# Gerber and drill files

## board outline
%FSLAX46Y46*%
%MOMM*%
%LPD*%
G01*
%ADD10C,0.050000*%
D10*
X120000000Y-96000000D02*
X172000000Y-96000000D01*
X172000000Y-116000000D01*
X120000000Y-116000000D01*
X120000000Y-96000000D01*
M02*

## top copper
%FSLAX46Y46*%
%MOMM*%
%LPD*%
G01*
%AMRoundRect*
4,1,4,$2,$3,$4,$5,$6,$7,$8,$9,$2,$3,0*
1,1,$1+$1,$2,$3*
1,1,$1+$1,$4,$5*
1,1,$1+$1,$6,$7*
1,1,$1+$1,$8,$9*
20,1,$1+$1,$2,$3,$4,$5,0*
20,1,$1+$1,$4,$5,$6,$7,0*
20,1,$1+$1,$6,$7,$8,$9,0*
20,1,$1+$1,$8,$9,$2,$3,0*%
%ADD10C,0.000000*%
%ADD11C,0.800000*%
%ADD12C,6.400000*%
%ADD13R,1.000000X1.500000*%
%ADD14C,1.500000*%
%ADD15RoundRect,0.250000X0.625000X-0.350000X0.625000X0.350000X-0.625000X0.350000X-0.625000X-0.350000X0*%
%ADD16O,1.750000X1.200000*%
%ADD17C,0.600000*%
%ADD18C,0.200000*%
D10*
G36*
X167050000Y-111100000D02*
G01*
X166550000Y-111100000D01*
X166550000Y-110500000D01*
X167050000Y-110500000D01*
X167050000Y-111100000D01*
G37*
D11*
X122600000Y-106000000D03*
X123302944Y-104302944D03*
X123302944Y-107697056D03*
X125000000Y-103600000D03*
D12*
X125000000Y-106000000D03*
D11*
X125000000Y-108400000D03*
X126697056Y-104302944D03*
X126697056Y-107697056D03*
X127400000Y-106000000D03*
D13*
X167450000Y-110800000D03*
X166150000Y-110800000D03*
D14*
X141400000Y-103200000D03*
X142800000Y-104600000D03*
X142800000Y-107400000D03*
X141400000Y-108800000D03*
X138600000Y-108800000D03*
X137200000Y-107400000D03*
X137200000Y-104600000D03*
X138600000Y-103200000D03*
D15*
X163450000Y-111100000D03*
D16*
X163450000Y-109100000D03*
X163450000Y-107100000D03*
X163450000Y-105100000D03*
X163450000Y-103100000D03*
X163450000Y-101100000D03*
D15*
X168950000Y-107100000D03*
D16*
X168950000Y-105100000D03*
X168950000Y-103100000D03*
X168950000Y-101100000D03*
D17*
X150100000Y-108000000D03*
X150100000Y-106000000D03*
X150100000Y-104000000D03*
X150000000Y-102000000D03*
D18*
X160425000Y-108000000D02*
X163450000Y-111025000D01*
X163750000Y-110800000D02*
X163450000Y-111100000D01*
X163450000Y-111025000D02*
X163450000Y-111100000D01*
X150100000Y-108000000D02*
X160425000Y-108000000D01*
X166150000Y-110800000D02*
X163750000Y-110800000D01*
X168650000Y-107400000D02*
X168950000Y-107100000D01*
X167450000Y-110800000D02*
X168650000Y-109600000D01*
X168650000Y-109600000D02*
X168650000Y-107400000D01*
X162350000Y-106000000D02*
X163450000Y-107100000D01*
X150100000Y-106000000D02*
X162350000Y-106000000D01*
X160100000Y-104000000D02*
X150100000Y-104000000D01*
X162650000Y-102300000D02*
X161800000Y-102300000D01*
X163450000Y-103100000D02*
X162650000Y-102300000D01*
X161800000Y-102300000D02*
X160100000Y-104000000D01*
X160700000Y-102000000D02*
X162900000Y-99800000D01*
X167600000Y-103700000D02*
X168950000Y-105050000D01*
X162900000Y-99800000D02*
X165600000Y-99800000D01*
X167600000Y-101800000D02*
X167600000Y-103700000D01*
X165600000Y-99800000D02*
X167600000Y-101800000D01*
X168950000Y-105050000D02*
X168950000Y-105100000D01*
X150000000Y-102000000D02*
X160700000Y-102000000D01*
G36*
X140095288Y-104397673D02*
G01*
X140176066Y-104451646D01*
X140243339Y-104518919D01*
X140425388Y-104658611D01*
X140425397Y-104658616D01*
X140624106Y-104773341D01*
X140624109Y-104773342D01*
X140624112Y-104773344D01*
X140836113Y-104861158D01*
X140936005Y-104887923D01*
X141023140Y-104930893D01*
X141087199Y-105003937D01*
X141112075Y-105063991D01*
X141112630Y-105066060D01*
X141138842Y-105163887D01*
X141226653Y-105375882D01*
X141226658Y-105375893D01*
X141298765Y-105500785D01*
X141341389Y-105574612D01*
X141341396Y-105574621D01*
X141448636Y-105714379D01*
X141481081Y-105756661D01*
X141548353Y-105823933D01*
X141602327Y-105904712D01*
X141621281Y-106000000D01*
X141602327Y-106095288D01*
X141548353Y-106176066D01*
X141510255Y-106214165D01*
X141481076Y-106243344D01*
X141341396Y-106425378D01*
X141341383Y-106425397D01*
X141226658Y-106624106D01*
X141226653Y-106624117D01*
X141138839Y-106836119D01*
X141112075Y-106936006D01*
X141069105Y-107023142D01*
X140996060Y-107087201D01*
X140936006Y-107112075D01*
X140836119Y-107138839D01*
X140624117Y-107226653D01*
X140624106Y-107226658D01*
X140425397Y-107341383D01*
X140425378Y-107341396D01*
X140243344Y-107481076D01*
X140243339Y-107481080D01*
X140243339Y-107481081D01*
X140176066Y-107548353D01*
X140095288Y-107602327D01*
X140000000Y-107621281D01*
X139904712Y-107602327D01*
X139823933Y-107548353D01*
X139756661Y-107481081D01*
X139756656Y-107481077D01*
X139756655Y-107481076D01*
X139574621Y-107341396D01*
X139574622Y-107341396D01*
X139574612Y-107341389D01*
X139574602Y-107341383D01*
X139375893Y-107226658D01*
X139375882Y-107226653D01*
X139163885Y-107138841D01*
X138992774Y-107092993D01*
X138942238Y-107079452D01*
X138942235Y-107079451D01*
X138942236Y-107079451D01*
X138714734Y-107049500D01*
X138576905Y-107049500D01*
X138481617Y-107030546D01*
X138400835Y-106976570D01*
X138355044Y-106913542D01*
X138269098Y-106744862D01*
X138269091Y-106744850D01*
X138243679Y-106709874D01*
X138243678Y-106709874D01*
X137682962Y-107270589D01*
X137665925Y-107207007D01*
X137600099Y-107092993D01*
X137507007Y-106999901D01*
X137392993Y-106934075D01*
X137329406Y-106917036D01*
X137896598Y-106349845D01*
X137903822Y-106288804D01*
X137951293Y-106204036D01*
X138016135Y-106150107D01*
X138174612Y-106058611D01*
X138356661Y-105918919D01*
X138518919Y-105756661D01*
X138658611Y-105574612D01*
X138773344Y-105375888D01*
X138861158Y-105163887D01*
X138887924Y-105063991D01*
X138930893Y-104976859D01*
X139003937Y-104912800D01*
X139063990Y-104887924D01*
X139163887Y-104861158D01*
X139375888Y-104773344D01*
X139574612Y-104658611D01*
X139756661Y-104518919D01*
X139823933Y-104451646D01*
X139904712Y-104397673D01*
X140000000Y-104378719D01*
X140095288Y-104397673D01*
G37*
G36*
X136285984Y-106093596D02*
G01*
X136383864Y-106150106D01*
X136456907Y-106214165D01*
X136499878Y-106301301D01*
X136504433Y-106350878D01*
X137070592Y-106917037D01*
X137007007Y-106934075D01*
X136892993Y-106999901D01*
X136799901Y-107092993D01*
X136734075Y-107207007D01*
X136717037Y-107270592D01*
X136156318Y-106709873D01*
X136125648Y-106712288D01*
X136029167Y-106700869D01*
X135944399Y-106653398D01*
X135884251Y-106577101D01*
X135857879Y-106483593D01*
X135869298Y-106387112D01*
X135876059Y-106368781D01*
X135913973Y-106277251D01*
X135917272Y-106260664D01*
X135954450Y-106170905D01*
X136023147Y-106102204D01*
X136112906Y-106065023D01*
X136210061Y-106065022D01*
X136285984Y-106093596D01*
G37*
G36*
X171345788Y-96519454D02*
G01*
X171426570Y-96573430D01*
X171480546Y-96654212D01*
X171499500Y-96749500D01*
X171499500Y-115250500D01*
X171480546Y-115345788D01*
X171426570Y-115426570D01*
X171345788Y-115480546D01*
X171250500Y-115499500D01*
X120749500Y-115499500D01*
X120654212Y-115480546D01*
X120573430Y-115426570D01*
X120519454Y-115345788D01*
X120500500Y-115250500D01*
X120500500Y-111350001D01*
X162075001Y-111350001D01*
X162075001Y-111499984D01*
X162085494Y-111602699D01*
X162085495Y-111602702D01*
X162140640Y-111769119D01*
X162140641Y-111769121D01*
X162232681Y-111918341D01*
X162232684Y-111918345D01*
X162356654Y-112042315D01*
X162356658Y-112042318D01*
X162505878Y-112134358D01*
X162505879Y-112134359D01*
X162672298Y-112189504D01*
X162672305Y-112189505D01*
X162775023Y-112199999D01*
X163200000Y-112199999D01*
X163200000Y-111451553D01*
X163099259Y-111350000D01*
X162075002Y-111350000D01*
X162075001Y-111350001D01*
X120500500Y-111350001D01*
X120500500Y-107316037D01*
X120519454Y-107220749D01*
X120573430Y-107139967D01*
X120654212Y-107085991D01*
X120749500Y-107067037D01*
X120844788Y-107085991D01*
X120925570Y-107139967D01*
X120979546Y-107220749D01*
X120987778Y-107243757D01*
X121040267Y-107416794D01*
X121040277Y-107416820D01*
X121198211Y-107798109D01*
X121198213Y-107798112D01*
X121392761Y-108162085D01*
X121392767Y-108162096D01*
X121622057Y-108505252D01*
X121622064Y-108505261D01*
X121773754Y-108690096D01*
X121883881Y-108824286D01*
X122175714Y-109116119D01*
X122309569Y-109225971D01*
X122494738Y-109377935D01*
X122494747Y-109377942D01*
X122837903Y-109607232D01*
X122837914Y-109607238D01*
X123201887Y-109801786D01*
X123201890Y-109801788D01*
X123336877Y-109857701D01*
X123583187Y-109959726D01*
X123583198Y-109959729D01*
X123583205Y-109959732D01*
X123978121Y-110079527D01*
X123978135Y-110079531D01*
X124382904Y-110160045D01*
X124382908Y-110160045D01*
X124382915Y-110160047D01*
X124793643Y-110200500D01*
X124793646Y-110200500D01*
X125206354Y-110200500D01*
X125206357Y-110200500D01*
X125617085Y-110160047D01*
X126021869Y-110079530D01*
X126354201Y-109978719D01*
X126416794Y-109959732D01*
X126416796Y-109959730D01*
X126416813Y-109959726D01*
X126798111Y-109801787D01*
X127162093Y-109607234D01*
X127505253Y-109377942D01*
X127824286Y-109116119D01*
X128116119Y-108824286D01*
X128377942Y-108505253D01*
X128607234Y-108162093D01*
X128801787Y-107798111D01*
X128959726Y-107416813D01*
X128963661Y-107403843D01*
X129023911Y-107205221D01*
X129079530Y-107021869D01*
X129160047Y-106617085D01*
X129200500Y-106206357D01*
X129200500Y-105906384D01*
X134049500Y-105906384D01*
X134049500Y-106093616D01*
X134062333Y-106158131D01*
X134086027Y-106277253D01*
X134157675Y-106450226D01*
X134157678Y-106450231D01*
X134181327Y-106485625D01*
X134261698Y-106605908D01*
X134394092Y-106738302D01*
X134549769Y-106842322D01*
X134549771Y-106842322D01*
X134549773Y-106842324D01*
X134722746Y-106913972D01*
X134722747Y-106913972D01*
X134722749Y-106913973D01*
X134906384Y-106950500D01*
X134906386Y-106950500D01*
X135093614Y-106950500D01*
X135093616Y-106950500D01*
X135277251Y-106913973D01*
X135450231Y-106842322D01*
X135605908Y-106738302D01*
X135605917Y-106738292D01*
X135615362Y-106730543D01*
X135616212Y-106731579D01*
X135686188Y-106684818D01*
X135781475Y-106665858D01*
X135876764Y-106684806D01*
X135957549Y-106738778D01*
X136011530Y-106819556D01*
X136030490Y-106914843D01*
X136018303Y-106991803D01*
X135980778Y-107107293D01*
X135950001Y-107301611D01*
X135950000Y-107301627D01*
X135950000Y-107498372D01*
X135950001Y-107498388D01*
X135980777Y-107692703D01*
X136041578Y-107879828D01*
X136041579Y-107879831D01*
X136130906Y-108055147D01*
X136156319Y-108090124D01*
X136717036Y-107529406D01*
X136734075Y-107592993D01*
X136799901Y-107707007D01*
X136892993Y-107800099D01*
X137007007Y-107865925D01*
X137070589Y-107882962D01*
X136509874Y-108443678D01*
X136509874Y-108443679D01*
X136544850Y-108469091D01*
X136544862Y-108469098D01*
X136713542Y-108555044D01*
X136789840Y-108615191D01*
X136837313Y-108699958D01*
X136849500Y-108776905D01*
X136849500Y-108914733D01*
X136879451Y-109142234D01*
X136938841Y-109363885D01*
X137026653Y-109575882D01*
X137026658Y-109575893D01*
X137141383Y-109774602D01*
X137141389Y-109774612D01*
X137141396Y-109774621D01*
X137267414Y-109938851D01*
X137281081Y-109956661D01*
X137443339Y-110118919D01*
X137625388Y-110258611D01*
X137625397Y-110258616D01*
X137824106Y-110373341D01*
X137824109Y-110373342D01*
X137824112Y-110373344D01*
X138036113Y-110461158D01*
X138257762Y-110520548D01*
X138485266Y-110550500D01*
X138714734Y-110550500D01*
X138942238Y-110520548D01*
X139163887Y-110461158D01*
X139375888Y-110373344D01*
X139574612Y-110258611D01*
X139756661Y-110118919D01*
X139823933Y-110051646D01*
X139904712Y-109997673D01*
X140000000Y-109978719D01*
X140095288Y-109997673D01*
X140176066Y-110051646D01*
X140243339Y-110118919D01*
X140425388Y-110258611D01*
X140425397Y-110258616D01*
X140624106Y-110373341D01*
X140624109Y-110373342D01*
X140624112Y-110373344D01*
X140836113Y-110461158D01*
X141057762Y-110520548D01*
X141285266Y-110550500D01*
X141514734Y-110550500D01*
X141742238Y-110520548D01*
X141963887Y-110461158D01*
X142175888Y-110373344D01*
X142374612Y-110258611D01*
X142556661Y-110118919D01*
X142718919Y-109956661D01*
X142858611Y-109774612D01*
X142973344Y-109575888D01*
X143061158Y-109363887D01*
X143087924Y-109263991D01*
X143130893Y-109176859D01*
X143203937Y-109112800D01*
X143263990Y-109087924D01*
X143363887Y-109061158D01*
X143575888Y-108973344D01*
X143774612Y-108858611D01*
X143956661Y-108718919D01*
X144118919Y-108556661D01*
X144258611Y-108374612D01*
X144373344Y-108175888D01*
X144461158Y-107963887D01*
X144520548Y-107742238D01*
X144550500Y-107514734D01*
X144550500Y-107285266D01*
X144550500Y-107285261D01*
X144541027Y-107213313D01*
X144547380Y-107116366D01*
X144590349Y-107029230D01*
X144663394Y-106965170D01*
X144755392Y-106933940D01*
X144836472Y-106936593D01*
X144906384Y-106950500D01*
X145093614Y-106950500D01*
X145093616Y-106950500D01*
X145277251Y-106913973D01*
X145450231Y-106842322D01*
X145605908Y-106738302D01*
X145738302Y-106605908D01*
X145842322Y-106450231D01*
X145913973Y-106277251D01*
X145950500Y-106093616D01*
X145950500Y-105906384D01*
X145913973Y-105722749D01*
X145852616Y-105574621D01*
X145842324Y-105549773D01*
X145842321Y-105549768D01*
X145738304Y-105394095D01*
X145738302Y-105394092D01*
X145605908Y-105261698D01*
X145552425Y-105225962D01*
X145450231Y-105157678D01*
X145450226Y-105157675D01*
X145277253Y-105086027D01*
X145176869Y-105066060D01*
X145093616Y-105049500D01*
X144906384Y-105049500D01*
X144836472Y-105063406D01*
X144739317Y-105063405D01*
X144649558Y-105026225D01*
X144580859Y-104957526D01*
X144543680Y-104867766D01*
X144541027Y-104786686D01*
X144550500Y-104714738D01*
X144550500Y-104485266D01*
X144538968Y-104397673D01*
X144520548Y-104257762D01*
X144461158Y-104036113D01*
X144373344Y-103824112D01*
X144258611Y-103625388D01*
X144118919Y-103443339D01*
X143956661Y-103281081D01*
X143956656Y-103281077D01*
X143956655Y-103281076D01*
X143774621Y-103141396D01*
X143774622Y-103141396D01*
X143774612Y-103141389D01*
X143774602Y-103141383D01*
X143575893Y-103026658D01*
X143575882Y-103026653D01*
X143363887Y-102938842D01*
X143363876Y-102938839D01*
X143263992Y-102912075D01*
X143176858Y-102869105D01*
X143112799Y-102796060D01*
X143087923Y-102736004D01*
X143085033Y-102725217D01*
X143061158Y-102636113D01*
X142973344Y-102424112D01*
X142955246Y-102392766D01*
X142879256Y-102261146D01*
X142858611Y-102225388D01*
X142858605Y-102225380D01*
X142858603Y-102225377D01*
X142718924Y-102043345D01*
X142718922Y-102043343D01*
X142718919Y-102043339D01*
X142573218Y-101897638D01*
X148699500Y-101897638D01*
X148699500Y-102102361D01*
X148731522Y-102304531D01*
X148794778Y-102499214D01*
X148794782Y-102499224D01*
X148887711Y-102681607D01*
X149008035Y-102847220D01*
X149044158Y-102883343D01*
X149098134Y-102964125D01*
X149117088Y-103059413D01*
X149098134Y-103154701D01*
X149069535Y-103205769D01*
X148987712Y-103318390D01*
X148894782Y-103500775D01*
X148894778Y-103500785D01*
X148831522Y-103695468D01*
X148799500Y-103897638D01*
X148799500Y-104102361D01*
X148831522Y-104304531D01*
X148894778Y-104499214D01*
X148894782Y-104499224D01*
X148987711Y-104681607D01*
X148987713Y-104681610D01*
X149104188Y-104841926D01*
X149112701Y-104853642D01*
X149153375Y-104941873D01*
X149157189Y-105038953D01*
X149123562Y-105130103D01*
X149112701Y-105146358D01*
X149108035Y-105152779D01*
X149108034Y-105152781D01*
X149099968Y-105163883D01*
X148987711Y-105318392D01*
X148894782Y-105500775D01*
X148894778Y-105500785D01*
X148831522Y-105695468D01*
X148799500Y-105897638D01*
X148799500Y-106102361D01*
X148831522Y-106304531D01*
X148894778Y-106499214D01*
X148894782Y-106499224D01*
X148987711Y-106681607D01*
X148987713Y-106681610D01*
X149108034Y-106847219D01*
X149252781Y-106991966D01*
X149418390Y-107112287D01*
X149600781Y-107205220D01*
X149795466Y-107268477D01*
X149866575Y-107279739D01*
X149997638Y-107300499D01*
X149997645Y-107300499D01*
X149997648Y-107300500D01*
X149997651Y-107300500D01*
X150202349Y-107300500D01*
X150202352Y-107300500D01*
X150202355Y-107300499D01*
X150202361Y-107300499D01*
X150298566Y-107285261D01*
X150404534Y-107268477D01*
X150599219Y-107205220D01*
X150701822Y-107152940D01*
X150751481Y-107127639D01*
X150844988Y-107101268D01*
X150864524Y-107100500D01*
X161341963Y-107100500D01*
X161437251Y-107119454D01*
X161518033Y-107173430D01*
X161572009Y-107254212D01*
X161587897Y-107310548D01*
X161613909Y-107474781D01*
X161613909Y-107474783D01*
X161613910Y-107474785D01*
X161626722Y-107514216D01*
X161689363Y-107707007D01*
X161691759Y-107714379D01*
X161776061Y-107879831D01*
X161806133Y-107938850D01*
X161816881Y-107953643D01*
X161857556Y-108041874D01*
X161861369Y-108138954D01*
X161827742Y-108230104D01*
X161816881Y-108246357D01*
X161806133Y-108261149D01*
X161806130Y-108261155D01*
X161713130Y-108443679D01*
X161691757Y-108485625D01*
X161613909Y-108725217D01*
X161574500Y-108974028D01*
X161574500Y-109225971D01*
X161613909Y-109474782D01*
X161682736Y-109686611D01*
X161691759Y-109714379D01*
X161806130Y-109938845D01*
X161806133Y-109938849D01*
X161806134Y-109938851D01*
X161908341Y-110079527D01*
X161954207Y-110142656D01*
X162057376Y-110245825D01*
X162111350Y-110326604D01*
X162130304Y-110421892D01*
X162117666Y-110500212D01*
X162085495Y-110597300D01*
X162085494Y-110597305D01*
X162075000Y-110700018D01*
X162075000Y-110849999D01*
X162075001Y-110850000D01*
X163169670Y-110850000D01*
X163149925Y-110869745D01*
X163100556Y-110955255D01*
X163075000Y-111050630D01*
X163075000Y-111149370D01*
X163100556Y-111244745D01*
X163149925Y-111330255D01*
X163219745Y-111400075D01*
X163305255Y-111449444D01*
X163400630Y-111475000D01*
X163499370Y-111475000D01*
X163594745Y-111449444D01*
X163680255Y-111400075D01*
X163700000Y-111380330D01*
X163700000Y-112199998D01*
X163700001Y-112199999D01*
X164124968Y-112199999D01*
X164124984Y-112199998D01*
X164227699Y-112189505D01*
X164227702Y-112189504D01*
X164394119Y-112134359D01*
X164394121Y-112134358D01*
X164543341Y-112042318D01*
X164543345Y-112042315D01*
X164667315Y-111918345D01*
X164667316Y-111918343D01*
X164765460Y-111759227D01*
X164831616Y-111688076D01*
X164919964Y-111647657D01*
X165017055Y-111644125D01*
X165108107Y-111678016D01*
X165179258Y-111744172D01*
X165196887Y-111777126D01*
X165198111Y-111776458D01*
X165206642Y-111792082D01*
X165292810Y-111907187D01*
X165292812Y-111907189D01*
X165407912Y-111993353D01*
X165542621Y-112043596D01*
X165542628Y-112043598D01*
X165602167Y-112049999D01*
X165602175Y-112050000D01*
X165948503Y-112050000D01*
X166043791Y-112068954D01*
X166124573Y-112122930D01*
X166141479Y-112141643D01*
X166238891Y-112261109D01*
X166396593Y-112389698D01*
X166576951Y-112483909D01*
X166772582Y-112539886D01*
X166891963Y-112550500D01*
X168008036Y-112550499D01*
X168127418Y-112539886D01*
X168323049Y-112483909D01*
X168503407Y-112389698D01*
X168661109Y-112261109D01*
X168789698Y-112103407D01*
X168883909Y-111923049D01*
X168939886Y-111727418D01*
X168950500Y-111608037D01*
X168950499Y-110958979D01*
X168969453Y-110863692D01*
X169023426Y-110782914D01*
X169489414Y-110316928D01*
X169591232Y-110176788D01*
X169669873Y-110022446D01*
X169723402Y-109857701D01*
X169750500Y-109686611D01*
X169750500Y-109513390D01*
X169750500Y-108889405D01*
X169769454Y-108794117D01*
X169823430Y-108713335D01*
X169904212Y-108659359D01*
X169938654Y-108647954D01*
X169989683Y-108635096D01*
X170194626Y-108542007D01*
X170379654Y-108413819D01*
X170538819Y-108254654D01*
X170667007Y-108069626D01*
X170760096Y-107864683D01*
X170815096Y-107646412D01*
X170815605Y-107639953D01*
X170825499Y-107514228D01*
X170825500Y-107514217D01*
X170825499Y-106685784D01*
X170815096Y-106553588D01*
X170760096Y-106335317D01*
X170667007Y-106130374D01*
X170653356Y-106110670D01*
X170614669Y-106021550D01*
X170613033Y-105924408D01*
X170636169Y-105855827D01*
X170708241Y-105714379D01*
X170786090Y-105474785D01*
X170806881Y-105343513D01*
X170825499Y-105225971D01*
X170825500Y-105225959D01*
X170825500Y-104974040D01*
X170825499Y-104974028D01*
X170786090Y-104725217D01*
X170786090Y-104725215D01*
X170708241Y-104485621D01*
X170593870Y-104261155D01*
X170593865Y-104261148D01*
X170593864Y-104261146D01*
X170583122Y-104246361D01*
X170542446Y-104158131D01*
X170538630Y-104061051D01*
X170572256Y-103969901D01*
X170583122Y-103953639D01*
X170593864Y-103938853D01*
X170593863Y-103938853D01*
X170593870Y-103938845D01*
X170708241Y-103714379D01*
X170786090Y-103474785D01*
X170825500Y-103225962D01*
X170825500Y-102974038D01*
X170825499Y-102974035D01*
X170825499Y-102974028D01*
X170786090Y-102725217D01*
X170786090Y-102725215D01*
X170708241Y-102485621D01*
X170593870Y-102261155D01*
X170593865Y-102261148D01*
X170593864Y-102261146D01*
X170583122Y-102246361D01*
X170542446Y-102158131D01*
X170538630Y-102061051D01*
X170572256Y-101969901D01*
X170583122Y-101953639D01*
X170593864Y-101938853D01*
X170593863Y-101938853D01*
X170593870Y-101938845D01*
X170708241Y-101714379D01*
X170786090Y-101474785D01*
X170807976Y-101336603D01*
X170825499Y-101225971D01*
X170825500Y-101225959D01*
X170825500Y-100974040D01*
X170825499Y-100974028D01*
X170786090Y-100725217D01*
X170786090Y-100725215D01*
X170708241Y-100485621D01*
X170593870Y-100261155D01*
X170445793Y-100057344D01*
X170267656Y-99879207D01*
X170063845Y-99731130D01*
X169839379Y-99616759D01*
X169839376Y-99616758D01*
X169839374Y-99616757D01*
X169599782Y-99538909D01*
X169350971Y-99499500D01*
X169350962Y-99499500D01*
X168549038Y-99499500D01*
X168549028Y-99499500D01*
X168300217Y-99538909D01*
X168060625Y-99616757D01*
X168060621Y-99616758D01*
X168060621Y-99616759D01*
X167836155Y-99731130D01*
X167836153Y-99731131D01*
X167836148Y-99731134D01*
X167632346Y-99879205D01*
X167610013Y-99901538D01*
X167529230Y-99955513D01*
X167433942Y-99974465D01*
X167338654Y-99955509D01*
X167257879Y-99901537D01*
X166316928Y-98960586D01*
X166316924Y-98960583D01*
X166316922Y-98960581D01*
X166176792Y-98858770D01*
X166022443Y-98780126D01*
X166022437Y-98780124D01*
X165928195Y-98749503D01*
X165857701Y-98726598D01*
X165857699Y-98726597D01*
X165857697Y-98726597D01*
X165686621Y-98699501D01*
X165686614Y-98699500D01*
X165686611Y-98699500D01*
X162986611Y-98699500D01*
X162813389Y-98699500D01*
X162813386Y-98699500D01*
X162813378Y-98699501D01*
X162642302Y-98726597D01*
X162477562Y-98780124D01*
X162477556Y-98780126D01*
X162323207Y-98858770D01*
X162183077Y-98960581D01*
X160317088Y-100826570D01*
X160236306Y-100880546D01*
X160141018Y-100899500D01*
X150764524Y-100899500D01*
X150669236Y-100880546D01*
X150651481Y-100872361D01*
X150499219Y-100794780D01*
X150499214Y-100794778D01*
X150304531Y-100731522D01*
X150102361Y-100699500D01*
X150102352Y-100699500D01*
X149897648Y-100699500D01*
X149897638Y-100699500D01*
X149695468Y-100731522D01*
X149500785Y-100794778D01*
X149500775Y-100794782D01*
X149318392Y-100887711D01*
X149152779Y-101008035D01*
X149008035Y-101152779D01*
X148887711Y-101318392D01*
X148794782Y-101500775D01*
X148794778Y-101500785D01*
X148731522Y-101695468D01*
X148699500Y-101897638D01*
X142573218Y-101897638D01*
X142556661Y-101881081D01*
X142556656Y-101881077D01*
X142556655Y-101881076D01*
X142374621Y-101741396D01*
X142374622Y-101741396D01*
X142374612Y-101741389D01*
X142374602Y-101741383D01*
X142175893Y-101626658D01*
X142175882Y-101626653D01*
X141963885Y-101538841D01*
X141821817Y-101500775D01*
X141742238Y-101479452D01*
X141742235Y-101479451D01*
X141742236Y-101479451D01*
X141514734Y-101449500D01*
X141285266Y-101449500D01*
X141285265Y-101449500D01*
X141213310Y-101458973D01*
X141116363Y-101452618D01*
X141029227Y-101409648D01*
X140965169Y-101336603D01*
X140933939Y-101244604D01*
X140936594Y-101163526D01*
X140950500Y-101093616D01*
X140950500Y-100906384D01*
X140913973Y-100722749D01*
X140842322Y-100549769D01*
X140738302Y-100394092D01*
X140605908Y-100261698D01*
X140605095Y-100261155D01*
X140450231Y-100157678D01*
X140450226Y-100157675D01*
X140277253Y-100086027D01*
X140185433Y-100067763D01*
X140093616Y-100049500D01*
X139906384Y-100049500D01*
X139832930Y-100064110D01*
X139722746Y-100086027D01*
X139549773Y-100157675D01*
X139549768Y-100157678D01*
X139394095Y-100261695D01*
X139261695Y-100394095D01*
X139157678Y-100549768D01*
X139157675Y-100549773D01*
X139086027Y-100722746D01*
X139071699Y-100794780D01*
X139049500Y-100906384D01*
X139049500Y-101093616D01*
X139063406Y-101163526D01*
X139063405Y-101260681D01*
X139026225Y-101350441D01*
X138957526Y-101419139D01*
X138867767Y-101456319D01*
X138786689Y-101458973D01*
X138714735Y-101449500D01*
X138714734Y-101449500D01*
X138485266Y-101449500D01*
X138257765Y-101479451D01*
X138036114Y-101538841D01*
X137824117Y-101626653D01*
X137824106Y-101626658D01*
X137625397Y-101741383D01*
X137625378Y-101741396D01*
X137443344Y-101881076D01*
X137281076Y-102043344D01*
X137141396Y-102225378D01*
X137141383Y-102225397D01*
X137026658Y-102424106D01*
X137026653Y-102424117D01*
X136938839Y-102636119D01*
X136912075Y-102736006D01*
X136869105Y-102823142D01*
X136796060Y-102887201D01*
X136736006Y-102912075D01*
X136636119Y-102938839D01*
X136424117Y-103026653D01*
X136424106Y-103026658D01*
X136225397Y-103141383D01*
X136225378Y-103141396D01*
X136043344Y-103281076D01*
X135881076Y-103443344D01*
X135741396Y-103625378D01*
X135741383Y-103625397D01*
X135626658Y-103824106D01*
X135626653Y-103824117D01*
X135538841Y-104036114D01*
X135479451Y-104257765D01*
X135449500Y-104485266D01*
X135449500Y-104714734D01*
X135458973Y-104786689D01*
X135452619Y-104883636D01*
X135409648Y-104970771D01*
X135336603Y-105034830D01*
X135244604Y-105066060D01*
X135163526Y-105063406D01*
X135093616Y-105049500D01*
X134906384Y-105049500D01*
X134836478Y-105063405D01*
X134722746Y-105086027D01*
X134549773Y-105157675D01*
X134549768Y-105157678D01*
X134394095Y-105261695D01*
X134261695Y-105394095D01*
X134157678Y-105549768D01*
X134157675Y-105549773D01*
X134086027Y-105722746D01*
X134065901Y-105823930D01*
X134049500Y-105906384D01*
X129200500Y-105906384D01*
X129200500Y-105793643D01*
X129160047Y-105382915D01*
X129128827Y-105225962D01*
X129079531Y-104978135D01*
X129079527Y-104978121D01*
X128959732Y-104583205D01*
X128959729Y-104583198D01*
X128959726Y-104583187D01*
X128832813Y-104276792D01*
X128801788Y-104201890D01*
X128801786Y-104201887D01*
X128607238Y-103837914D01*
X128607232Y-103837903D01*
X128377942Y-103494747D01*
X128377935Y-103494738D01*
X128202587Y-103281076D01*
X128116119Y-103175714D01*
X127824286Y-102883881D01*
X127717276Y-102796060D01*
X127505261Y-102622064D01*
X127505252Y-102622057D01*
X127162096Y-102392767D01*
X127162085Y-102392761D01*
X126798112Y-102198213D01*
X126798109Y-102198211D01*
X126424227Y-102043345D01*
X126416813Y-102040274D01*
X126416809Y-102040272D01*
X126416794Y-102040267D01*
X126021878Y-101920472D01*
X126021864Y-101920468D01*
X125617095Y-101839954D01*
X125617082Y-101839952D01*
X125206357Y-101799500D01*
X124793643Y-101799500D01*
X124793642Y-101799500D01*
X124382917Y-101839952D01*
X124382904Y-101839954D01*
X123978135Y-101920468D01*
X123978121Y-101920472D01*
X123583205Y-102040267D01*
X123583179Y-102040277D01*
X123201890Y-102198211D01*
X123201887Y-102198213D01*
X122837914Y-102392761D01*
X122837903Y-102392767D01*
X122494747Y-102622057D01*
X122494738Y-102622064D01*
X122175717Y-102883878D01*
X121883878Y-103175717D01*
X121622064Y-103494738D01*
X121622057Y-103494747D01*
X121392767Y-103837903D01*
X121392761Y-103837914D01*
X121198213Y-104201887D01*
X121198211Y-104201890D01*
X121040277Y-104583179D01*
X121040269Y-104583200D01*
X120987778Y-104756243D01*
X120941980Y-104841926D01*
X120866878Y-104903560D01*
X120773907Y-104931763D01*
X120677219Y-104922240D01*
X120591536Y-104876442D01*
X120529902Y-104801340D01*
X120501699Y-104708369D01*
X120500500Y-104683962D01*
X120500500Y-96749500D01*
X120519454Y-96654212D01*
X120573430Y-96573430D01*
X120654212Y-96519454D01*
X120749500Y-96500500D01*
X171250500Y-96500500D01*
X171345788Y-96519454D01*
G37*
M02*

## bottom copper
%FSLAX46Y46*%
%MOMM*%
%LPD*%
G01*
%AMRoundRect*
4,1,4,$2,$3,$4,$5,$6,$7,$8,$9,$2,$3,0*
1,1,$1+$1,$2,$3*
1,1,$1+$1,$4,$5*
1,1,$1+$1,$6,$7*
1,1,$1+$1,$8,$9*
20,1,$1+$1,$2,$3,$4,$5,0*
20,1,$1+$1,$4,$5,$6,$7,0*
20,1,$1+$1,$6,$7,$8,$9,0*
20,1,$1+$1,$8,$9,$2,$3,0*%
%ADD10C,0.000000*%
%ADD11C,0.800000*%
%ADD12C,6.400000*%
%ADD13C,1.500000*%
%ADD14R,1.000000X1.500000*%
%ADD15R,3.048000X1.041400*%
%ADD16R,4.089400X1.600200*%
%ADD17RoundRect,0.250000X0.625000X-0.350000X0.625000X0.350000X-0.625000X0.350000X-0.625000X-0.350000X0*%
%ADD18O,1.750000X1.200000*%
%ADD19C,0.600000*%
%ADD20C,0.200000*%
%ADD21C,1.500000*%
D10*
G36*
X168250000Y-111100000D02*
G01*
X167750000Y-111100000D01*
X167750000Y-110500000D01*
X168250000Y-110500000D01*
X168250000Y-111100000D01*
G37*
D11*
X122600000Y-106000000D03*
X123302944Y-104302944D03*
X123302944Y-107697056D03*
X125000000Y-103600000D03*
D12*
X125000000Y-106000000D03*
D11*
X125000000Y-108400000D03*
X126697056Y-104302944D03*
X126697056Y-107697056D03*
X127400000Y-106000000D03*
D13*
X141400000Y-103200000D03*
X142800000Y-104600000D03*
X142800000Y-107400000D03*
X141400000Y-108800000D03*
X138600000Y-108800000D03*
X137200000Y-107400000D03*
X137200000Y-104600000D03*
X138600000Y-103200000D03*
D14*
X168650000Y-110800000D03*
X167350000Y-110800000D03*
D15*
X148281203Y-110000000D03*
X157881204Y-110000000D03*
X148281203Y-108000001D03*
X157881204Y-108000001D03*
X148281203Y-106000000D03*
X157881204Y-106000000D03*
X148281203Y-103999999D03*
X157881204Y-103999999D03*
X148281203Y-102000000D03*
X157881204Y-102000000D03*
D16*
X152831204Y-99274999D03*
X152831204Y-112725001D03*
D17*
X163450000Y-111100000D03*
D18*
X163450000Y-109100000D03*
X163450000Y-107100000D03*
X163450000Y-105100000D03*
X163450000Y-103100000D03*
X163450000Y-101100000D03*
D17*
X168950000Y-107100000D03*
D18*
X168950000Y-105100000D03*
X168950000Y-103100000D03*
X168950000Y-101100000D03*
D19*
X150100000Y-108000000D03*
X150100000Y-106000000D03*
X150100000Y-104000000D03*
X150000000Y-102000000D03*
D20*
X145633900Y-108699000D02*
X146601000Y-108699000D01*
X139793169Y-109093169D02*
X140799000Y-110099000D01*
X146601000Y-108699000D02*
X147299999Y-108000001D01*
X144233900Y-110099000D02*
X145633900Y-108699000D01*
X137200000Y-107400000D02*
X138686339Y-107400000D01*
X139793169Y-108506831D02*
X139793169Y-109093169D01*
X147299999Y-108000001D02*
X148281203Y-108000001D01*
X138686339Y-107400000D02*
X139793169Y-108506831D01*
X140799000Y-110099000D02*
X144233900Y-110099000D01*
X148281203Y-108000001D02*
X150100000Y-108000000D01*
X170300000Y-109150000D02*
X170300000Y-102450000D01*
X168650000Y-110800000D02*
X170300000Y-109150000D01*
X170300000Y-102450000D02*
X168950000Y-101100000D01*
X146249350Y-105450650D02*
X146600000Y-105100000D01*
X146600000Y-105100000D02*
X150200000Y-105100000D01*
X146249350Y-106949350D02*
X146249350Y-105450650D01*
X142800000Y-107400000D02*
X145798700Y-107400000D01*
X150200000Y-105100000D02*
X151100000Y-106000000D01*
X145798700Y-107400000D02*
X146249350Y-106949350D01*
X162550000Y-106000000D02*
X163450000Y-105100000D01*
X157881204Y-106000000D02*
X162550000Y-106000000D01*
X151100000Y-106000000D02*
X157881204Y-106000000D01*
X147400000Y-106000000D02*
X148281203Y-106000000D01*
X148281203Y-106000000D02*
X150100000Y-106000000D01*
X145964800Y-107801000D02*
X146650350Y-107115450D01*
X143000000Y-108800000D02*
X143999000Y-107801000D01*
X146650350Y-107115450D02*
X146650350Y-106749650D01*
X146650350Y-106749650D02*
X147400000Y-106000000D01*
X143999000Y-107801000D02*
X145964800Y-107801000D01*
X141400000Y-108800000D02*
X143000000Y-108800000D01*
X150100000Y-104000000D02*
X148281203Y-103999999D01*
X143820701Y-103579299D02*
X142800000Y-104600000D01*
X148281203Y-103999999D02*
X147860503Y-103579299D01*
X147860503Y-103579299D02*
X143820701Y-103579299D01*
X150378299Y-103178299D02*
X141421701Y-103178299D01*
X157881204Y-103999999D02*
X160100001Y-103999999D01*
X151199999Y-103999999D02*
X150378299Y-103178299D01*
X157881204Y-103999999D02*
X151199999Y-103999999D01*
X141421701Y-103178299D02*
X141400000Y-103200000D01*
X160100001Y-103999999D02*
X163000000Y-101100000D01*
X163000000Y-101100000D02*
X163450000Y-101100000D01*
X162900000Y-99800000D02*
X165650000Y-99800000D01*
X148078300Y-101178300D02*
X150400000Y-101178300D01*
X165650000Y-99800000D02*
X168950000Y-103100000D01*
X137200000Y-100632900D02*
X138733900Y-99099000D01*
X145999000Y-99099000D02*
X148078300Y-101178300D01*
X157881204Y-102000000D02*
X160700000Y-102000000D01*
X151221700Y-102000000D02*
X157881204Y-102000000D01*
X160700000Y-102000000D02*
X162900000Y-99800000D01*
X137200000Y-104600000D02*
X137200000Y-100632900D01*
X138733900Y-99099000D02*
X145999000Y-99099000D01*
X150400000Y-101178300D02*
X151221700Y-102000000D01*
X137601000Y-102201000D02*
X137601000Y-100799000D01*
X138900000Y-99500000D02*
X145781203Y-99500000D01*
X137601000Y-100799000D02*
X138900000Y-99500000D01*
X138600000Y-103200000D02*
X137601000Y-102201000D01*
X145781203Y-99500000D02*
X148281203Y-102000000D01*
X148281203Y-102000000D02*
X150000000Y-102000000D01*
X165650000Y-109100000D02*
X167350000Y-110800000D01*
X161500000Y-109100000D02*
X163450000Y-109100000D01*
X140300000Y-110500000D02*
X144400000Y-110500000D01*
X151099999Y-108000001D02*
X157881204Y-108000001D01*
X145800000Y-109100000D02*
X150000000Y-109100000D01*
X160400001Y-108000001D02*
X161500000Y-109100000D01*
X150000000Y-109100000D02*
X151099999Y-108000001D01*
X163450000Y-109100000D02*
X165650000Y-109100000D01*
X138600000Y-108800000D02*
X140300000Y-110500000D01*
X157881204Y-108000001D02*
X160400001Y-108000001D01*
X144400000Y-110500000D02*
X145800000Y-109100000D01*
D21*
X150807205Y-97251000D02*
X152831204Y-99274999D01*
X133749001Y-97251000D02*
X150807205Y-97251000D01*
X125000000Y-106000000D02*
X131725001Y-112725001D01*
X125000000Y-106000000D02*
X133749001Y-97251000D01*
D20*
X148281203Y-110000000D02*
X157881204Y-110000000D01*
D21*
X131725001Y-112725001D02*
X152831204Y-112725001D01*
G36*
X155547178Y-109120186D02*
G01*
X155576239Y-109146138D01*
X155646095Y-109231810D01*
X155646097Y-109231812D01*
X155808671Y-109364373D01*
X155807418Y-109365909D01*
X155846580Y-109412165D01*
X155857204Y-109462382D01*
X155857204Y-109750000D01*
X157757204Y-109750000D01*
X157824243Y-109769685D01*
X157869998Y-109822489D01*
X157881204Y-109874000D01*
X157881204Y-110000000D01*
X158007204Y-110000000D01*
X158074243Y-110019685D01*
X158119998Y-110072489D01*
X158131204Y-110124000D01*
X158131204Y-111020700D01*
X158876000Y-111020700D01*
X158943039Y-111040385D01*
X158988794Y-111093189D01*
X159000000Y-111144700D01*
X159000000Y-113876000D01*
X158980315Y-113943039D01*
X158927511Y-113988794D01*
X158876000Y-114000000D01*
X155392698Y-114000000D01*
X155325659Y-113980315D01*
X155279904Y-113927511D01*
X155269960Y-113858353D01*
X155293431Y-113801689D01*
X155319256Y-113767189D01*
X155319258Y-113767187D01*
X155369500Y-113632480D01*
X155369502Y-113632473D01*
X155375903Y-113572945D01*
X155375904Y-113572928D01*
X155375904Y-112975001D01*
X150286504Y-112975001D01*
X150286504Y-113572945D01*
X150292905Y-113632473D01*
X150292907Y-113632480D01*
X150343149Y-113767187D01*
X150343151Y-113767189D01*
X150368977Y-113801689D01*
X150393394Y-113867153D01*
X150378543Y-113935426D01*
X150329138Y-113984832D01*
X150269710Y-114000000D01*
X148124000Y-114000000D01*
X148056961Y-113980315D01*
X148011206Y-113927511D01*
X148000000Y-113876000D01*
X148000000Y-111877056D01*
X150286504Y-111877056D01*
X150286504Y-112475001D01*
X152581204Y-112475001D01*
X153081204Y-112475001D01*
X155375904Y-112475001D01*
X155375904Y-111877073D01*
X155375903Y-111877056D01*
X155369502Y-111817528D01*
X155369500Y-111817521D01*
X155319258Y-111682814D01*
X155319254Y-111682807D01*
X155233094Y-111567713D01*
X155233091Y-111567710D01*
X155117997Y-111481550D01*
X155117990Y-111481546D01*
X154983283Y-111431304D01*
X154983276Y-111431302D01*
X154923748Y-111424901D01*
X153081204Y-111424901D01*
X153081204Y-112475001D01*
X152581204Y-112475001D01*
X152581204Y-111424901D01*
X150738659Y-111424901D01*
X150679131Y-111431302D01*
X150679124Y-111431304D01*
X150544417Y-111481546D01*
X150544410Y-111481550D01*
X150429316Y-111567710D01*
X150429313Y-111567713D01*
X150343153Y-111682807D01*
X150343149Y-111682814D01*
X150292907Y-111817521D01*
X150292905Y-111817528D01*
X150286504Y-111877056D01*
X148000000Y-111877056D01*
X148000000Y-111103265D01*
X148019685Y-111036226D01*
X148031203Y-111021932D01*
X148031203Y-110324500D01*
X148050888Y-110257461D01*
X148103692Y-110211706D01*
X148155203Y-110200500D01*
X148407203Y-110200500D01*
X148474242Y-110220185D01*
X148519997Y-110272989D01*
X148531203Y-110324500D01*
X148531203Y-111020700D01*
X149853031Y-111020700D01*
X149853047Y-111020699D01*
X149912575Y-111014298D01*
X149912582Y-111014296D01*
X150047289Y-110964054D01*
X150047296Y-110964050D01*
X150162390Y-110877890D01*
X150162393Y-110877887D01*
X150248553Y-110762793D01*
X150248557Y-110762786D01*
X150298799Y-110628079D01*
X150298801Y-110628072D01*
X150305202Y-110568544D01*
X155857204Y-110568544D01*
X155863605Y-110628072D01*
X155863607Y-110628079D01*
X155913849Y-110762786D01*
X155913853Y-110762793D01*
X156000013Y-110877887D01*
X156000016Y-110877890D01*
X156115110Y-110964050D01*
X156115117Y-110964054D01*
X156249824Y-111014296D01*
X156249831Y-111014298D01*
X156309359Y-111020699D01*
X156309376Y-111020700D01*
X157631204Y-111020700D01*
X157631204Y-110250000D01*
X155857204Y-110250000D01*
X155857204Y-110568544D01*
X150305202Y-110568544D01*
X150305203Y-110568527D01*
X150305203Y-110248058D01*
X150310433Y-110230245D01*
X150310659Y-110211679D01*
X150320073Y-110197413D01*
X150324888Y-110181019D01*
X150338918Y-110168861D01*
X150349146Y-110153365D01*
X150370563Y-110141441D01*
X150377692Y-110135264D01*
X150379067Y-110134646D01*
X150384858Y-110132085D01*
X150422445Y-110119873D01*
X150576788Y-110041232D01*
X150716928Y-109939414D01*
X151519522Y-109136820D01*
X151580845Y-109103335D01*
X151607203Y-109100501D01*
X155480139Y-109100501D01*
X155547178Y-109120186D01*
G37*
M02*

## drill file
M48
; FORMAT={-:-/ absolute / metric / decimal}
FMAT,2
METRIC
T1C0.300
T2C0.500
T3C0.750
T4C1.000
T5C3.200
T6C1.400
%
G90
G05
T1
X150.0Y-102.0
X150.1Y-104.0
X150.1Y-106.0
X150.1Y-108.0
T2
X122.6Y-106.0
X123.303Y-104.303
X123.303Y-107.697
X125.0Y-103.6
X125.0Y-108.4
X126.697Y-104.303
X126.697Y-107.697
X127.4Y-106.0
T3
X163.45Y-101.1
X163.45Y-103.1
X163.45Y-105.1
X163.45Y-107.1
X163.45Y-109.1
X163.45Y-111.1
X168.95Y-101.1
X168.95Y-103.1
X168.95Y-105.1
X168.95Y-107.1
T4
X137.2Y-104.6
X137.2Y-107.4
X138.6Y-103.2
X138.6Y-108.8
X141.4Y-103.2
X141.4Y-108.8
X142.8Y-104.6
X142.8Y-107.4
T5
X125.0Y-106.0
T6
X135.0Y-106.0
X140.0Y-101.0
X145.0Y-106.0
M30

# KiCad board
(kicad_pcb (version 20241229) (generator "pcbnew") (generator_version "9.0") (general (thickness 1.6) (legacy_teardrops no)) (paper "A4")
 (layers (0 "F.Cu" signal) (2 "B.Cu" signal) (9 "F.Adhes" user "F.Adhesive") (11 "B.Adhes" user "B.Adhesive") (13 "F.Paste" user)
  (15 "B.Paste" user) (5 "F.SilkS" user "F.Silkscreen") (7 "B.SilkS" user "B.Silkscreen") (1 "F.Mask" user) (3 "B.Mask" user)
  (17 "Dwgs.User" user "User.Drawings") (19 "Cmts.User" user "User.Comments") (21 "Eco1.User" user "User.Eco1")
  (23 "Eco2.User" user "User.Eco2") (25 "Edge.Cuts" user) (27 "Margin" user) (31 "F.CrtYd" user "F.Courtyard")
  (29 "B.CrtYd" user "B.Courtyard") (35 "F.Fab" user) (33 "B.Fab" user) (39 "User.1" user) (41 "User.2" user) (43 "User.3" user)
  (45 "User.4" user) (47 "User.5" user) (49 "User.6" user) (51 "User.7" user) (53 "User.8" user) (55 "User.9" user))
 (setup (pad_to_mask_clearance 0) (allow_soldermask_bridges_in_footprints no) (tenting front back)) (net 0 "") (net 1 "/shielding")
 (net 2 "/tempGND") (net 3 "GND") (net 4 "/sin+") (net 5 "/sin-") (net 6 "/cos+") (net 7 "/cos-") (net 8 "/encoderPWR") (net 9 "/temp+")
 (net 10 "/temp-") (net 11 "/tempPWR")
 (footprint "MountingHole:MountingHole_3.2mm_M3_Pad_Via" (layer "F.Cu") (at 125 106)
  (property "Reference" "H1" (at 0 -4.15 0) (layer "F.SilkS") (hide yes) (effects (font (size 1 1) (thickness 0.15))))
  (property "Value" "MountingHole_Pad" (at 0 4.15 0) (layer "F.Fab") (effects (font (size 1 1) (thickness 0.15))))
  (pad "1" thru_hole circle (at -2.4 0) (size 0.8 0.8) (drill 0.5) (layers "*.Cu" "*.Mask") (remove_unused_layers no) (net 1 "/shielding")
   (zone_connect 2))
  (pad "1" thru_hole circle (at -1.697056 -1.697056) (size 0.8 0.8) (drill 0.5) (layers "*.Cu" "*.Mask") (remove_unused_layers no)
   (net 1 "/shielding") (zone_connect 2))
  (pad "1" thru_hole circle (at -1.697056 1.697056) (size 0.8 0.8) (drill 0.5) (layers "*.Cu" "*.Mask") (remove_unused_layers no)
   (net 1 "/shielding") (zone_connect 2))
  (pad "1" thru_hole circle (at 0 -2.4) (size 0.8 0.8) (drill 0.5) (layers "*.Cu" "*.Mask") (remove_unused_layers no) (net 1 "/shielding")
   (zone_connect 2))
  (pad "1" thru_hole circle (at 0 0) (size 6.4 6.4) (drill 3.2) (layers "*.Cu" "*.Mask") (remove_unused_layers no) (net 1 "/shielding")
   (zone_connect 2))
  (pad "1" thru_hole circle (at 0 2.4) (size 0.8 0.8) (drill 0.5) (layers "*.Cu" "*.Mask") (remove_unused_layers no) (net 1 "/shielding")
   (zone_connect 2))
  (pad "1" thru_hole circle (at 1.697056 -1.697056) (size 0.8 0.8) (drill 0.5) (layers "*.Cu" "*.Mask") (remove_unused_layers no)
   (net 1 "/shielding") (zone_connect 2))
  (pad "1" thru_hole circle (at 1.697056 1.697056) (size 0.8 0.8) (drill 0.5) (layers "*.Cu" "*.Mask") (remove_unused_layers no)
   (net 1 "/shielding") (zone_connect 2))
  (pad "1" thru_hole circle (at 2.4 0) (size 0.8 0.8) (drill 0.5) (layers "*.Cu" "*.Mask") (remove_unused_layers no) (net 1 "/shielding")
   (zone_connect 2)))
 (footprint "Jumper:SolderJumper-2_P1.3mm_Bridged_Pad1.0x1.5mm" (layer "F.Cu") (at 166.8 110.8 180)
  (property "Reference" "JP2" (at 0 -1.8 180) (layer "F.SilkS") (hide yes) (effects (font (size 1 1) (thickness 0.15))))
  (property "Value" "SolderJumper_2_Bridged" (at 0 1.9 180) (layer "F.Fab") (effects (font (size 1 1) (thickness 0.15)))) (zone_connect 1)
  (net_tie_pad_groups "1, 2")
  (fp_poly (pts (xy -0.25 -0.3) (xy 0.25 -0.3) (xy 0.25 0.3) (xy -0.25 0.3)) (stroke (width 0) (type solid)) (fill yes) (layer "F.Cu"))
  (pad "1" smd rect (at -0.65 0 180) (size 1 1.5) (layers "F.Cu" "F.Mask") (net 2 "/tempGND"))
  (pad "2" smd rect (at 0.65 0 180) (size 1 1.5) (layers "F.Cu" "F.Mask") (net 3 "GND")))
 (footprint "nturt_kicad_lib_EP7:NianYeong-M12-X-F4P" (layer "F.Cu") (at 140 106 -90)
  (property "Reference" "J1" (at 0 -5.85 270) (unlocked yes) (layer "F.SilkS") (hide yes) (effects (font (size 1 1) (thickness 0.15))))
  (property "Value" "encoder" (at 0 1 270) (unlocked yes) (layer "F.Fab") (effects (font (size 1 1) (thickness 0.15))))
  (pad "" np_thru_hole circle (at -5 0 270) (size 1.4 1.4) (drill 1.4) (layers "*.Cu" "*.Mask"))
  (pad "" np_thru_hole circle (at 0 -5 270) (size 1.4 1.4) (drill 1.4) (layers "*.Cu" "*.Mask"))
  (pad "" np_thru_hole circle (at 0 5 270) (size 1.4 1.4) (drill 1.4) (layers "*.Cu" "*.Mask"))
  (pad "1" thru_hole circle (at -2.8 -1.4 270) (size 1.5 1.5) (drill 1) (layers "*.Cu" "*.Mask") (remove_unused_layers no) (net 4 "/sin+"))
  (pad "2" thru_hole circle (at -1.4 -2.8 270) (size 1.5 1.5) (drill 1) (layers "*.Cu" "*.Mask") (remove_unused_layers no) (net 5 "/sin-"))
  (pad "3" thru_hole circle (at 1.4 -2.8 270) (size 1.5 1.5) (drill 1) (layers "*.Cu" "*.Mask") (remove_unused_layers no) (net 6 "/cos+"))
  (pad "4" thru_hole circle (at 2.8 -1.4 270) (size 1.5 1.5) (drill 1) (layers "*.Cu" "*.Mask") (remove_unused_layers no) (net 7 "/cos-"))
  (pad "5" thru_hole circle (at 2.8 1.4 270) (size 1.5 1.5) (drill 1) (layers "*.Cu" "*.Mask") (remove_unused_layers no)
   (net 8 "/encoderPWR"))
  (pad "6" thru_hole circle (at 1.4 2.8 270) (size 1.5 1.5) (drill 1) (layers "*.Cu" "*.Mask") (remove_unused_layers no) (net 3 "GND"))
  (pad "7" thru_hole circle (at -1.4 2.8 270) (size 1.5 1.5) (drill 1) (layers "*.Cu" "*.Mask") (remove_unused_layers no) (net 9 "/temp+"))
  (pad "8" thru_hole circle (at -2.8 1.4 270) (size 1.5 1.5) (drill 1) (layers "*.Cu" "*.Mask") (remove_unused_layers no) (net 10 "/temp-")))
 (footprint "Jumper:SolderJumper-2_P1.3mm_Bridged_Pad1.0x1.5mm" (layer "B.Cu") (at 168 110.8 180)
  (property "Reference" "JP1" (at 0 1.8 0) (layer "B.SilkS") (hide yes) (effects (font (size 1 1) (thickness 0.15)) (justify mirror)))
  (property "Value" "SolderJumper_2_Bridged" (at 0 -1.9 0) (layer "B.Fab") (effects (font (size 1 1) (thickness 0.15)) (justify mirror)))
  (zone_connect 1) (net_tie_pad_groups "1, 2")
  (fp_poly (pts (xy -0.25 0.3) (xy 0.25 0.3) (xy 0.25 -0.3) (xy -0.25 -0.3)) (stroke (width 0) (type solid)) (fill yes) (layer "B.Cu"))
  (pad "1" smd rect (at -0.65 0 180) (size 1 1.5) (layers "B.Cu" "B.Mask") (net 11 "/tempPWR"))
  (pad "2" smd rect (at 0.65 0 180) (size 1 1.5) (layers "B.Cu" "B.Mask") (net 8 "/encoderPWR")))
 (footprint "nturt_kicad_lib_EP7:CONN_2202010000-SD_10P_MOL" (layer "B.Cu") (at 152.8 106 -90)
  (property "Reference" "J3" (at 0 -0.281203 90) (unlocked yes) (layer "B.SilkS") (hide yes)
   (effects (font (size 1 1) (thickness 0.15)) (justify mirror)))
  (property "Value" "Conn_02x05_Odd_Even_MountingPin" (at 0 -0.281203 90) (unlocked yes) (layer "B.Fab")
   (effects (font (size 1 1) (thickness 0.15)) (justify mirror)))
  (pad "1" smd rect (at 4 4.518797 270) (size 1.0414 3.048) (layers "B.Cu" "B.Mask" "B.Paste") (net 1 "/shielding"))
  (pad "2" smd rect (at 4 -5.081204 270) (size 1.0414 3.048) (layers "B.Cu" "B.Mask" "B.Paste") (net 1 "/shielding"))
  (pad "3" smd rect (at 2.000001 4.518797 270) (size 1.0414 3.048) (layers "B.Cu" "B.Mask" "B.Paste") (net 3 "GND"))
  (pad "4" smd rect (at 2.000001 -5.081204 270) (size 1.0414 3.048) (layers "B.Cu" "B.Mask" "B.Paste") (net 8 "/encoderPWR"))
  (pad "5" smd rect (at 0 4.518797 270) (size 1.0414 3.048) (layers "B.Cu" "B.Mask" "B.Paste") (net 7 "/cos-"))
  (pad "6" smd rect (at 0 -5.081204 270) (size 1.0414 3.048) (layers "B.Cu" "B.Mask" "B.Paste") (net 6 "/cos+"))
  (pad "7" smd rect (at -2.000001 4.518797 270) (size 1.0414 3.048) (layers "B.Cu" "B.Mask" "B.Paste") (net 5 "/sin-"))
  (pad "8" smd rect (at -2.000001 -5.081204 270) (size 1.0414 3.048) (layers "B.Cu" "B.Mask" "B.Paste") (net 4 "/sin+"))
  (pad "9" smd rect (at -4 4.518797 270) (size 1.0414 3.048) (layers "B.Cu" "B.Mask" "B.Paste") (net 10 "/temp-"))
  (pad "10" smd rect (at -4 -5.081204 270) (size 1.0414 3.048) (layers "B.Cu" "B.Mask" "B.Paste") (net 9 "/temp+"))
  (pad "MP" smd rect (at -6.725001 -0.031204 270) (size 1.6002 4.0894) (layers "B.Cu" "B.Mask" "B.Paste") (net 1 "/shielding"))
  (pad "MP" smd rect (at 6.725001 -0.031204 270) (size 1.6002 4.0894) (layers "B.Cu" "B.Mask" "B.Paste") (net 1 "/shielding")))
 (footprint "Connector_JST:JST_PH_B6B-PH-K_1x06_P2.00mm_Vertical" (layer "B.Cu") (at 163.45 111.1 90)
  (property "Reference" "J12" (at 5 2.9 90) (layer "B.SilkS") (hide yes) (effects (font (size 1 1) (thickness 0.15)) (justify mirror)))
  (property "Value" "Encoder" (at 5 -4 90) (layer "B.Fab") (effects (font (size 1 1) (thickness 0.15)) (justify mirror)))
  (pad "1" thru_hole roundrect (at 0 0 90) (size 1.2 1.75) (drill 0.75) (layers "*.Cu" "*.Mask") (remove_unused_layers no)
   (roundrect_rratio 0.208333) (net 3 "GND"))
  (pad "2" thru_hole oval (at 2 0 90) (size 1.2 1.75) (drill 0.75) (layers "*.Cu" "*.Mask") (remove_unused_layers no) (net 8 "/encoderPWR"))
  (pad "3" thru_hole oval (at 4 0 90) (size 1.2 1.75) (drill 0.75) (layers "*.Cu" "*.Mask") (remove_unused_layers no) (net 7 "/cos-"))
  (pad "4" thru_hole oval (at 6 0 90) (size 1.2 1.75) (drill 0.75) (layers "*.Cu" "*.Mask") (remove_unused_layers no) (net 6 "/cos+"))
  (pad "5" thru_hole oval (at 8 0 90) (size 1.2 1.75) (drill 0.75) (layers "*.Cu" "*.Mask") (remove_unused_layers no) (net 5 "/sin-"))
  (pad "6" thru_hole oval (at 10 0 90) (size 1.2 1.75) (drill 0.75) (layers "*.Cu" "*.Mask") (remove_unused_layers no) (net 4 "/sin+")))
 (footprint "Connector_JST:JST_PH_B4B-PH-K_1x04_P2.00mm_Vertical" (layer "B.Cu") (at 168.95 107.1 90)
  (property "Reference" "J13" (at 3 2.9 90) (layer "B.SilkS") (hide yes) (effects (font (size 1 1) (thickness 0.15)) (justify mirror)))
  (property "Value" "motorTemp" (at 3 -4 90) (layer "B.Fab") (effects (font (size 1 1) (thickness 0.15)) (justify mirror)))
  (pad "1" thru_hole roundrect (at 0 0 90) (size 1.2 1.75) (drill 0.75) (layers "*.Cu" "*.Mask") (remove_unused_layers no)
   (roundrect_rratio 0.208333) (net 2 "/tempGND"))
  (pad "2" thru_hole oval (at 2 0 90) (size 1.2 1.75) (drill 0.75) (layers "*.Cu" "*.Mask") (remove_unused_layers no) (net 10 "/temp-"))
  (pad "3" thru_hole oval (at 4 0 90) (size 1.2 1.75) (drill 0.75) (layers "*.Cu" "*.Mask") (remove_unused_layers no) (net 9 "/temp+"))
  (pad "4" thru_hole oval (at 6 0 90) (size 1.2 1.75) (drill 0.75) (layers "*.Cu" "*.Mask") (remove_unused_layers no) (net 11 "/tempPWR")))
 (gr_rect (start 120 96) (end 172 116) (stroke (width 0.05) (type default)) (fill no) (layer "Edge.Cuts"))
 (segment (start 160.425 108) (end 163.45 111.025) (width 0.2) (layer "F.Cu") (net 3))
 (segment (start 163.75 110.8) (end 163.45 111.1) (width 0.2) (layer "F.Cu") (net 3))
 (segment (start 163.45 111.025) (end 163.45 111.1) (width 0.2) (layer "F.Cu") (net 3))
 (segment (start 150.1 108) (end 160.425 108) (width 0.2) (layer "F.Cu") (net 3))
 (segment (start 166.15 110.8) (end 163.75 110.8) (width 0.2) (layer "F.Cu") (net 3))
 (via (at 150.1 108) (size 0.6) (drill 0.3) (layers "F.Cu" "B.Cu") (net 3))
 (segment (start 145.6339 108.699) (end 146.601 108.699) (width 0.2) (layer "B.Cu") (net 3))
 (segment (start 139.793169 109.093169) (end 140.799 110.099) (width 0.2) (layer "B.Cu") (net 3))
 (segment (start 146.601 108.699) (end 147.299999 108.000001) (width 0.2) (layer "B.Cu") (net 3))
 (segment (start 144.2339 110.099) (end 145.6339 108.699) (width 0.2) (layer "B.Cu") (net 3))
 (segment (start 137.2 107.4) (end 138.686339 107.4) (width 0.2) (layer "B.Cu") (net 3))
 (segment (start 139.793169 108.506831) (end 139.793169 109.093169) (width 0.2) (layer "B.Cu") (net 3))
 (segment (start 147.299999 108.000001) (end 148.281203 108.000001) (width 0.2) (layer "B.Cu") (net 3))
 (segment (start 138.686339 107.4) (end 139.793169 108.506831) (width 0.2) (layer "B.Cu") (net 3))
 (segment (start 140.799 110.099) (end 144.2339 110.099) (width 0.2) (layer "B.Cu") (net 3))
 (segment (start 148.281203 108.000001) (end 150.1 108) (width 0.2) (layer "B.Cu") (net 3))
 (segment (start 170.3 109.15) (end 170.3 102.45) (width 0.2) (layer "B.Cu") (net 11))
 (segment (start 168.65 110.8) (end 170.3 109.15) (width 0.2) (layer "B.Cu") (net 11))
 (segment (start 170.3 102.45) (end 168.95 101.1) (width 0.2) (layer "B.Cu") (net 11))
 (segment (start 168.65 107.4) (end 168.95 107.1) (width 0.2) (layer "F.Cu") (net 2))
 (segment (start 167.45 110.8) (end 168.65 109.6) (width 0.2) (layer "F.Cu") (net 2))
 (segment (start 168.65 109.6) (end 168.65 107.4) (width 0.2) (layer "F.Cu") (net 2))
 (segment (start 146.24935 105.45065) (end 146.6 105.1) (width 0.2) (layer "B.Cu") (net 6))
 (segment (start 146.6 105.1) (end 150.2 105.1) (width 0.2) (layer "B.Cu") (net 6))
 (segment (start 146.24935 106.94935) (end 146.24935 105.45065) (width 0.2) (layer "B.Cu") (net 6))
 (segment (start 142.8 107.4) (end 145.7987 107.4) (width 0.2) (layer "B.Cu") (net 6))
 (segment (start 150.2 105.1) (end 151.1 106) (width 0.2) (layer "B.Cu") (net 6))
 (segment (start 145.7987 107.4) (end 146.24935 106.94935) (width 0.2) (layer "B.Cu") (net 6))
 (segment (start 162.55 106) (end 163.45 105.1) (width 0.2) (layer "B.Cu") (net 6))
 (segment (start 157.881204 106) (end 162.55 106) (width 0.2) (layer "B.Cu") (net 6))
 (segment (start 151.1 106) (end 157.881204 106) (width 0.2) (layer "B.Cu") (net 6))
 (segment (start 162.35 106) (end 163.45 107.1) (width 0.2) (layer "F.Cu") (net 7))
 (segment (start 150.1 106) (end 162.35 106) (width 0.2) (layer "F.Cu") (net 7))
 (via (at 150.1 106) (size 0.6) (drill 0.3) (layers "F.Cu" "B.Cu") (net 7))
 (segment (start 147.4 106) (end 148.281203 106) (width 0.2) (layer "B.Cu") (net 7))
 (segment (start 148.281203 106) (end 150.1 106) (width 0.2) (layer "B.Cu") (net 7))
 (segment (start 145.9648 107.801) (end 146.65035 107.11545) (width 0.2) (layer "B.Cu") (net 7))
 (segment (start 143 108.8) (end 143.999 107.801) (width 0.2) (layer "B.Cu") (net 7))
 (segment (start 146.65035 107.11545) (end 146.65035 106.74965) (width 0.2) (layer "B.Cu") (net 7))
 (segment (start 146.65035 106.74965) (end 147.4 106) (width 0.2) (layer "B.Cu") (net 7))
 (segment (start 143.999 107.801) (end 145.9648 107.801) (width 0.2) (layer "B.Cu") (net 7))
 (segment (start 141.4 108.8) (end 143 108.8) (width 0.2) (layer "B.Cu") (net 7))
 (segment (start 160.1 104) (end 150.1 104) (width 0.2) (layer "F.Cu") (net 5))
 (segment (start 162.65 102.3) (end 161.8 102.3) (width 0.2) (layer "F.Cu") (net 5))
 (segment (start 163.45 103.1) (end 162.65 102.3) (width 0.2) (layer "F.Cu") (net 5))
 (segment (start 161.8 102.3) (end 160.1 104) (width 0.2) (layer "F.Cu") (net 5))
 (via (at 150.1 104) (size 0.6) (drill 0.3) (layers "F.Cu" "B.Cu") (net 5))
 (segment (start 150.1 104) (end 148.281203 103.999999) (width 0.2) (layer "B.Cu") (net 5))
 (segment (start 143.820701 103.579299) (end 142.8 104.6) (width 0.2) (layer "B.Cu") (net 5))
 (segment (start 148.281203 103.999999) (end 147.860503 103.579299) (width 0.2) (layer "B.Cu") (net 5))
 (segment (start 147.860503 103.579299) (end 143.820701 103.579299) (width 0.2) (layer "B.Cu") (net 5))
 (segment (start 150.378299 103.178299) (end 141.421701 103.178299) (width 0.2) (layer "B.Cu") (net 4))
 (segment (start 157.881204 103.999999) (end 160.100001 103.999999) (width 0.2) (layer "B.Cu") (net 4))
 (segment (start 151.199999 103.999999) (end 150.378299 103.178299) (width 0.2) (layer "B.Cu") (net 4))
 (segment (start 157.881204 103.999999) (end 151.199999 103.999999) (width 0.2) (layer "B.Cu") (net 4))
 (segment (start 141.421701 103.178299) (end 141.4 103.2) (width 0.2) (layer "B.Cu") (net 4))
 (segment (start 160.100001 103.999999) (end 163 101.1) (width 0.2) (layer "B.Cu") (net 4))
 (segment (start 163 101.1) (end 163.45 101.1) (width 0.2) (layer "B.Cu") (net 4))
 (segment (start 162.9 99.8) (end 165.65 99.8) (width 0.2) (layer "B.Cu") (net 9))
 (segment (start 148.0783 101.1783) (end 150.4 101.1783) (width 0.2) (layer "B.Cu") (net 9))
 (segment (start 165.65 99.8) (end 168.95 103.1) (width 0.2) (layer "B.Cu") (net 9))
 (segment (start 137.2 100.6329) (end 138.7339 99.099) (width 0.2) (layer "B.Cu") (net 9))
 (segment (start 145.999 99.099) (end 148.0783 101.1783) (width 0.2) (layer "B.Cu") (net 9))
 (segment (start 157.881204 102) (end 160.7 102) (width 0.2) (layer "B.Cu") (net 9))
 (segment (start 151.2217 102) (end 157.881204 102) (width 0.2) (layer "B.Cu") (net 9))
 (segment (start 160.7 102) (end 162.9 99.8) (width 0.2) (layer "B.Cu") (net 9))
 (segment (start 137.2 104.6) (end 137.2 100.6329) (width 0.2) (layer "B.Cu") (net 9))
 (segment (start 138.7339 99.099) (end 145.999 99.099) (width 0.2) (layer "B.Cu") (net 9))
 (segment (start 150.4 101.1783) (end 151.2217 102) (width 0.2) (layer "B.Cu") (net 9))
 (segment (start 160.7 102) (end 162.9 99.8) (width 0.2) (layer "F.Cu") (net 10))
 (segment (start 167.6 103.7) (end 168.95 105.05) (width 0.2) (layer "F.Cu") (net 10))
 (segment (start 162.9 99.8) (end 165.6 99.8) (width 0.2) (layer "F.Cu") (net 10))
 (segment (start 167.6 101.8) (end 167.6 103.7) (width 0.2) (layer "F.Cu") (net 10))
 (segment (start 165.6 99.8) (end 167.6 101.8) (width 0.2) (layer "F.Cu") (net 10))
 (segment (start 168.95 105.05) (end 168.95 105.1) (width 0.2) (layer "F.Cu") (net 10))
 (segment (start 150 102) (end 160.7 102) (width 0.2) (layer "F.Cu") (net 10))
 (via (at 150 102) (size 0.6) (drill 0.3) (layers "F.Cu" "B.Cu") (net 10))
 (segment (start 137.601 102.201) (end 137.601 100.799) (width 0.2) (layer "B.Cu") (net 10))
 (segment (start 138.9 99.5) (end 145.781203 99.5) (width 0.2) (layer "B.Cu") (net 10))
 (segment (start 137.601 100.799) (end 138.9 99.5) (width 0.2) (layer "B.Cu") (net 10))
 (segment (start 138.6 103.2) (end 137.601 102.201) (width 0.2) (layer "B.Cu") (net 10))
 (segment (start 145.781203 99.5) (end 148.281203 102) (width 0.2) (layer "B.Cu") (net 10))
 (segment (start 148.281203 102) (end 150 102) (width 0.2) (layer "B.Cu") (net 10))
 (segment (start 165.65 109.1) (end 167.35 110.8) (width 0.2) (layer "B.Cu") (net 8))
 (segment (start 161.5 109.1) (end 163.45 109.1) (width 0.2) (layer "B.Cu") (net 8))
 (segment (start 140.3 110.5) (end 144.4 110.5) (width 0.2) (layer "B.Cu") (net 8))
 (segment (start 151.099999 108.000001) (end 157.881204 108.000001) (width 0.2) (layer "B.Cu") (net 8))
 (segment (start 145.8 109.1) (end 150 109.1) (width 0.2) (layer "B.Cu") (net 8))
 (segment (start 160.400001 108.000001) (end 161.5 109.1) (width 0.2) (layer "B.Cu") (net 8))
 (segment (start 150 109.1) (end 151.099999 108.000001) (width 0.2) (layer "B.Cu") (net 8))
 (segment (start 163.45 109.1) (end 165.65 109.1) (width 0.2) (layer "B.Cu") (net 8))
 (segment (start 138.6 108.8) (end 140.3 110.5) (width 0.2) (layer "B.Cu") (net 8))
 (segment (start 157.881204 108.000001) (end 160.400001 108.000001) (width 0.2) (layer "B.Cu") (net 8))
 (segment (start 144.4 110.5) (end 145.8 109.1) (width 0.2) (layer "B.Cu") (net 8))
 (segment (start 150.807205 97.251) (end 152.831204 99.274999) (width 1.5) (layer "B.Cu") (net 1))
 (segment (start 133.749001 97.251) (end 150.807205 97.251) (width 1.5) (layer "B.Cu") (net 1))
 (segment (start 125 106) (end 131.725001 112.725001) (width 1.5) (layer "B.Cu") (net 1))
 (segment (start 125 106) (end 133.749001 97.251) (width 1.5) (layer "B.Cu") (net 1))
 (segment (start 148.281203 110) (end 157.881204 110) (width 0.2) (layer "B.Cu") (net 1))
 (segment (start 131.725001 112.725001) (end 152.831204 112.725001) (width 1.5) (layer "B.Cu") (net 1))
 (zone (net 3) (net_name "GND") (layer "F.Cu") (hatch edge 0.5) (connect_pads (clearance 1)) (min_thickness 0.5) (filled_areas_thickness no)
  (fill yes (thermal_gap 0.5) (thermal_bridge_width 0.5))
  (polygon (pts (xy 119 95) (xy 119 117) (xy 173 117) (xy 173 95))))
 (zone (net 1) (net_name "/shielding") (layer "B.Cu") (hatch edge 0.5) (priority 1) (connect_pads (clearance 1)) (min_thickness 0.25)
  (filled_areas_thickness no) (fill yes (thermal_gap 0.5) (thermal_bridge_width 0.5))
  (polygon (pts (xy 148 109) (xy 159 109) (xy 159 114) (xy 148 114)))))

